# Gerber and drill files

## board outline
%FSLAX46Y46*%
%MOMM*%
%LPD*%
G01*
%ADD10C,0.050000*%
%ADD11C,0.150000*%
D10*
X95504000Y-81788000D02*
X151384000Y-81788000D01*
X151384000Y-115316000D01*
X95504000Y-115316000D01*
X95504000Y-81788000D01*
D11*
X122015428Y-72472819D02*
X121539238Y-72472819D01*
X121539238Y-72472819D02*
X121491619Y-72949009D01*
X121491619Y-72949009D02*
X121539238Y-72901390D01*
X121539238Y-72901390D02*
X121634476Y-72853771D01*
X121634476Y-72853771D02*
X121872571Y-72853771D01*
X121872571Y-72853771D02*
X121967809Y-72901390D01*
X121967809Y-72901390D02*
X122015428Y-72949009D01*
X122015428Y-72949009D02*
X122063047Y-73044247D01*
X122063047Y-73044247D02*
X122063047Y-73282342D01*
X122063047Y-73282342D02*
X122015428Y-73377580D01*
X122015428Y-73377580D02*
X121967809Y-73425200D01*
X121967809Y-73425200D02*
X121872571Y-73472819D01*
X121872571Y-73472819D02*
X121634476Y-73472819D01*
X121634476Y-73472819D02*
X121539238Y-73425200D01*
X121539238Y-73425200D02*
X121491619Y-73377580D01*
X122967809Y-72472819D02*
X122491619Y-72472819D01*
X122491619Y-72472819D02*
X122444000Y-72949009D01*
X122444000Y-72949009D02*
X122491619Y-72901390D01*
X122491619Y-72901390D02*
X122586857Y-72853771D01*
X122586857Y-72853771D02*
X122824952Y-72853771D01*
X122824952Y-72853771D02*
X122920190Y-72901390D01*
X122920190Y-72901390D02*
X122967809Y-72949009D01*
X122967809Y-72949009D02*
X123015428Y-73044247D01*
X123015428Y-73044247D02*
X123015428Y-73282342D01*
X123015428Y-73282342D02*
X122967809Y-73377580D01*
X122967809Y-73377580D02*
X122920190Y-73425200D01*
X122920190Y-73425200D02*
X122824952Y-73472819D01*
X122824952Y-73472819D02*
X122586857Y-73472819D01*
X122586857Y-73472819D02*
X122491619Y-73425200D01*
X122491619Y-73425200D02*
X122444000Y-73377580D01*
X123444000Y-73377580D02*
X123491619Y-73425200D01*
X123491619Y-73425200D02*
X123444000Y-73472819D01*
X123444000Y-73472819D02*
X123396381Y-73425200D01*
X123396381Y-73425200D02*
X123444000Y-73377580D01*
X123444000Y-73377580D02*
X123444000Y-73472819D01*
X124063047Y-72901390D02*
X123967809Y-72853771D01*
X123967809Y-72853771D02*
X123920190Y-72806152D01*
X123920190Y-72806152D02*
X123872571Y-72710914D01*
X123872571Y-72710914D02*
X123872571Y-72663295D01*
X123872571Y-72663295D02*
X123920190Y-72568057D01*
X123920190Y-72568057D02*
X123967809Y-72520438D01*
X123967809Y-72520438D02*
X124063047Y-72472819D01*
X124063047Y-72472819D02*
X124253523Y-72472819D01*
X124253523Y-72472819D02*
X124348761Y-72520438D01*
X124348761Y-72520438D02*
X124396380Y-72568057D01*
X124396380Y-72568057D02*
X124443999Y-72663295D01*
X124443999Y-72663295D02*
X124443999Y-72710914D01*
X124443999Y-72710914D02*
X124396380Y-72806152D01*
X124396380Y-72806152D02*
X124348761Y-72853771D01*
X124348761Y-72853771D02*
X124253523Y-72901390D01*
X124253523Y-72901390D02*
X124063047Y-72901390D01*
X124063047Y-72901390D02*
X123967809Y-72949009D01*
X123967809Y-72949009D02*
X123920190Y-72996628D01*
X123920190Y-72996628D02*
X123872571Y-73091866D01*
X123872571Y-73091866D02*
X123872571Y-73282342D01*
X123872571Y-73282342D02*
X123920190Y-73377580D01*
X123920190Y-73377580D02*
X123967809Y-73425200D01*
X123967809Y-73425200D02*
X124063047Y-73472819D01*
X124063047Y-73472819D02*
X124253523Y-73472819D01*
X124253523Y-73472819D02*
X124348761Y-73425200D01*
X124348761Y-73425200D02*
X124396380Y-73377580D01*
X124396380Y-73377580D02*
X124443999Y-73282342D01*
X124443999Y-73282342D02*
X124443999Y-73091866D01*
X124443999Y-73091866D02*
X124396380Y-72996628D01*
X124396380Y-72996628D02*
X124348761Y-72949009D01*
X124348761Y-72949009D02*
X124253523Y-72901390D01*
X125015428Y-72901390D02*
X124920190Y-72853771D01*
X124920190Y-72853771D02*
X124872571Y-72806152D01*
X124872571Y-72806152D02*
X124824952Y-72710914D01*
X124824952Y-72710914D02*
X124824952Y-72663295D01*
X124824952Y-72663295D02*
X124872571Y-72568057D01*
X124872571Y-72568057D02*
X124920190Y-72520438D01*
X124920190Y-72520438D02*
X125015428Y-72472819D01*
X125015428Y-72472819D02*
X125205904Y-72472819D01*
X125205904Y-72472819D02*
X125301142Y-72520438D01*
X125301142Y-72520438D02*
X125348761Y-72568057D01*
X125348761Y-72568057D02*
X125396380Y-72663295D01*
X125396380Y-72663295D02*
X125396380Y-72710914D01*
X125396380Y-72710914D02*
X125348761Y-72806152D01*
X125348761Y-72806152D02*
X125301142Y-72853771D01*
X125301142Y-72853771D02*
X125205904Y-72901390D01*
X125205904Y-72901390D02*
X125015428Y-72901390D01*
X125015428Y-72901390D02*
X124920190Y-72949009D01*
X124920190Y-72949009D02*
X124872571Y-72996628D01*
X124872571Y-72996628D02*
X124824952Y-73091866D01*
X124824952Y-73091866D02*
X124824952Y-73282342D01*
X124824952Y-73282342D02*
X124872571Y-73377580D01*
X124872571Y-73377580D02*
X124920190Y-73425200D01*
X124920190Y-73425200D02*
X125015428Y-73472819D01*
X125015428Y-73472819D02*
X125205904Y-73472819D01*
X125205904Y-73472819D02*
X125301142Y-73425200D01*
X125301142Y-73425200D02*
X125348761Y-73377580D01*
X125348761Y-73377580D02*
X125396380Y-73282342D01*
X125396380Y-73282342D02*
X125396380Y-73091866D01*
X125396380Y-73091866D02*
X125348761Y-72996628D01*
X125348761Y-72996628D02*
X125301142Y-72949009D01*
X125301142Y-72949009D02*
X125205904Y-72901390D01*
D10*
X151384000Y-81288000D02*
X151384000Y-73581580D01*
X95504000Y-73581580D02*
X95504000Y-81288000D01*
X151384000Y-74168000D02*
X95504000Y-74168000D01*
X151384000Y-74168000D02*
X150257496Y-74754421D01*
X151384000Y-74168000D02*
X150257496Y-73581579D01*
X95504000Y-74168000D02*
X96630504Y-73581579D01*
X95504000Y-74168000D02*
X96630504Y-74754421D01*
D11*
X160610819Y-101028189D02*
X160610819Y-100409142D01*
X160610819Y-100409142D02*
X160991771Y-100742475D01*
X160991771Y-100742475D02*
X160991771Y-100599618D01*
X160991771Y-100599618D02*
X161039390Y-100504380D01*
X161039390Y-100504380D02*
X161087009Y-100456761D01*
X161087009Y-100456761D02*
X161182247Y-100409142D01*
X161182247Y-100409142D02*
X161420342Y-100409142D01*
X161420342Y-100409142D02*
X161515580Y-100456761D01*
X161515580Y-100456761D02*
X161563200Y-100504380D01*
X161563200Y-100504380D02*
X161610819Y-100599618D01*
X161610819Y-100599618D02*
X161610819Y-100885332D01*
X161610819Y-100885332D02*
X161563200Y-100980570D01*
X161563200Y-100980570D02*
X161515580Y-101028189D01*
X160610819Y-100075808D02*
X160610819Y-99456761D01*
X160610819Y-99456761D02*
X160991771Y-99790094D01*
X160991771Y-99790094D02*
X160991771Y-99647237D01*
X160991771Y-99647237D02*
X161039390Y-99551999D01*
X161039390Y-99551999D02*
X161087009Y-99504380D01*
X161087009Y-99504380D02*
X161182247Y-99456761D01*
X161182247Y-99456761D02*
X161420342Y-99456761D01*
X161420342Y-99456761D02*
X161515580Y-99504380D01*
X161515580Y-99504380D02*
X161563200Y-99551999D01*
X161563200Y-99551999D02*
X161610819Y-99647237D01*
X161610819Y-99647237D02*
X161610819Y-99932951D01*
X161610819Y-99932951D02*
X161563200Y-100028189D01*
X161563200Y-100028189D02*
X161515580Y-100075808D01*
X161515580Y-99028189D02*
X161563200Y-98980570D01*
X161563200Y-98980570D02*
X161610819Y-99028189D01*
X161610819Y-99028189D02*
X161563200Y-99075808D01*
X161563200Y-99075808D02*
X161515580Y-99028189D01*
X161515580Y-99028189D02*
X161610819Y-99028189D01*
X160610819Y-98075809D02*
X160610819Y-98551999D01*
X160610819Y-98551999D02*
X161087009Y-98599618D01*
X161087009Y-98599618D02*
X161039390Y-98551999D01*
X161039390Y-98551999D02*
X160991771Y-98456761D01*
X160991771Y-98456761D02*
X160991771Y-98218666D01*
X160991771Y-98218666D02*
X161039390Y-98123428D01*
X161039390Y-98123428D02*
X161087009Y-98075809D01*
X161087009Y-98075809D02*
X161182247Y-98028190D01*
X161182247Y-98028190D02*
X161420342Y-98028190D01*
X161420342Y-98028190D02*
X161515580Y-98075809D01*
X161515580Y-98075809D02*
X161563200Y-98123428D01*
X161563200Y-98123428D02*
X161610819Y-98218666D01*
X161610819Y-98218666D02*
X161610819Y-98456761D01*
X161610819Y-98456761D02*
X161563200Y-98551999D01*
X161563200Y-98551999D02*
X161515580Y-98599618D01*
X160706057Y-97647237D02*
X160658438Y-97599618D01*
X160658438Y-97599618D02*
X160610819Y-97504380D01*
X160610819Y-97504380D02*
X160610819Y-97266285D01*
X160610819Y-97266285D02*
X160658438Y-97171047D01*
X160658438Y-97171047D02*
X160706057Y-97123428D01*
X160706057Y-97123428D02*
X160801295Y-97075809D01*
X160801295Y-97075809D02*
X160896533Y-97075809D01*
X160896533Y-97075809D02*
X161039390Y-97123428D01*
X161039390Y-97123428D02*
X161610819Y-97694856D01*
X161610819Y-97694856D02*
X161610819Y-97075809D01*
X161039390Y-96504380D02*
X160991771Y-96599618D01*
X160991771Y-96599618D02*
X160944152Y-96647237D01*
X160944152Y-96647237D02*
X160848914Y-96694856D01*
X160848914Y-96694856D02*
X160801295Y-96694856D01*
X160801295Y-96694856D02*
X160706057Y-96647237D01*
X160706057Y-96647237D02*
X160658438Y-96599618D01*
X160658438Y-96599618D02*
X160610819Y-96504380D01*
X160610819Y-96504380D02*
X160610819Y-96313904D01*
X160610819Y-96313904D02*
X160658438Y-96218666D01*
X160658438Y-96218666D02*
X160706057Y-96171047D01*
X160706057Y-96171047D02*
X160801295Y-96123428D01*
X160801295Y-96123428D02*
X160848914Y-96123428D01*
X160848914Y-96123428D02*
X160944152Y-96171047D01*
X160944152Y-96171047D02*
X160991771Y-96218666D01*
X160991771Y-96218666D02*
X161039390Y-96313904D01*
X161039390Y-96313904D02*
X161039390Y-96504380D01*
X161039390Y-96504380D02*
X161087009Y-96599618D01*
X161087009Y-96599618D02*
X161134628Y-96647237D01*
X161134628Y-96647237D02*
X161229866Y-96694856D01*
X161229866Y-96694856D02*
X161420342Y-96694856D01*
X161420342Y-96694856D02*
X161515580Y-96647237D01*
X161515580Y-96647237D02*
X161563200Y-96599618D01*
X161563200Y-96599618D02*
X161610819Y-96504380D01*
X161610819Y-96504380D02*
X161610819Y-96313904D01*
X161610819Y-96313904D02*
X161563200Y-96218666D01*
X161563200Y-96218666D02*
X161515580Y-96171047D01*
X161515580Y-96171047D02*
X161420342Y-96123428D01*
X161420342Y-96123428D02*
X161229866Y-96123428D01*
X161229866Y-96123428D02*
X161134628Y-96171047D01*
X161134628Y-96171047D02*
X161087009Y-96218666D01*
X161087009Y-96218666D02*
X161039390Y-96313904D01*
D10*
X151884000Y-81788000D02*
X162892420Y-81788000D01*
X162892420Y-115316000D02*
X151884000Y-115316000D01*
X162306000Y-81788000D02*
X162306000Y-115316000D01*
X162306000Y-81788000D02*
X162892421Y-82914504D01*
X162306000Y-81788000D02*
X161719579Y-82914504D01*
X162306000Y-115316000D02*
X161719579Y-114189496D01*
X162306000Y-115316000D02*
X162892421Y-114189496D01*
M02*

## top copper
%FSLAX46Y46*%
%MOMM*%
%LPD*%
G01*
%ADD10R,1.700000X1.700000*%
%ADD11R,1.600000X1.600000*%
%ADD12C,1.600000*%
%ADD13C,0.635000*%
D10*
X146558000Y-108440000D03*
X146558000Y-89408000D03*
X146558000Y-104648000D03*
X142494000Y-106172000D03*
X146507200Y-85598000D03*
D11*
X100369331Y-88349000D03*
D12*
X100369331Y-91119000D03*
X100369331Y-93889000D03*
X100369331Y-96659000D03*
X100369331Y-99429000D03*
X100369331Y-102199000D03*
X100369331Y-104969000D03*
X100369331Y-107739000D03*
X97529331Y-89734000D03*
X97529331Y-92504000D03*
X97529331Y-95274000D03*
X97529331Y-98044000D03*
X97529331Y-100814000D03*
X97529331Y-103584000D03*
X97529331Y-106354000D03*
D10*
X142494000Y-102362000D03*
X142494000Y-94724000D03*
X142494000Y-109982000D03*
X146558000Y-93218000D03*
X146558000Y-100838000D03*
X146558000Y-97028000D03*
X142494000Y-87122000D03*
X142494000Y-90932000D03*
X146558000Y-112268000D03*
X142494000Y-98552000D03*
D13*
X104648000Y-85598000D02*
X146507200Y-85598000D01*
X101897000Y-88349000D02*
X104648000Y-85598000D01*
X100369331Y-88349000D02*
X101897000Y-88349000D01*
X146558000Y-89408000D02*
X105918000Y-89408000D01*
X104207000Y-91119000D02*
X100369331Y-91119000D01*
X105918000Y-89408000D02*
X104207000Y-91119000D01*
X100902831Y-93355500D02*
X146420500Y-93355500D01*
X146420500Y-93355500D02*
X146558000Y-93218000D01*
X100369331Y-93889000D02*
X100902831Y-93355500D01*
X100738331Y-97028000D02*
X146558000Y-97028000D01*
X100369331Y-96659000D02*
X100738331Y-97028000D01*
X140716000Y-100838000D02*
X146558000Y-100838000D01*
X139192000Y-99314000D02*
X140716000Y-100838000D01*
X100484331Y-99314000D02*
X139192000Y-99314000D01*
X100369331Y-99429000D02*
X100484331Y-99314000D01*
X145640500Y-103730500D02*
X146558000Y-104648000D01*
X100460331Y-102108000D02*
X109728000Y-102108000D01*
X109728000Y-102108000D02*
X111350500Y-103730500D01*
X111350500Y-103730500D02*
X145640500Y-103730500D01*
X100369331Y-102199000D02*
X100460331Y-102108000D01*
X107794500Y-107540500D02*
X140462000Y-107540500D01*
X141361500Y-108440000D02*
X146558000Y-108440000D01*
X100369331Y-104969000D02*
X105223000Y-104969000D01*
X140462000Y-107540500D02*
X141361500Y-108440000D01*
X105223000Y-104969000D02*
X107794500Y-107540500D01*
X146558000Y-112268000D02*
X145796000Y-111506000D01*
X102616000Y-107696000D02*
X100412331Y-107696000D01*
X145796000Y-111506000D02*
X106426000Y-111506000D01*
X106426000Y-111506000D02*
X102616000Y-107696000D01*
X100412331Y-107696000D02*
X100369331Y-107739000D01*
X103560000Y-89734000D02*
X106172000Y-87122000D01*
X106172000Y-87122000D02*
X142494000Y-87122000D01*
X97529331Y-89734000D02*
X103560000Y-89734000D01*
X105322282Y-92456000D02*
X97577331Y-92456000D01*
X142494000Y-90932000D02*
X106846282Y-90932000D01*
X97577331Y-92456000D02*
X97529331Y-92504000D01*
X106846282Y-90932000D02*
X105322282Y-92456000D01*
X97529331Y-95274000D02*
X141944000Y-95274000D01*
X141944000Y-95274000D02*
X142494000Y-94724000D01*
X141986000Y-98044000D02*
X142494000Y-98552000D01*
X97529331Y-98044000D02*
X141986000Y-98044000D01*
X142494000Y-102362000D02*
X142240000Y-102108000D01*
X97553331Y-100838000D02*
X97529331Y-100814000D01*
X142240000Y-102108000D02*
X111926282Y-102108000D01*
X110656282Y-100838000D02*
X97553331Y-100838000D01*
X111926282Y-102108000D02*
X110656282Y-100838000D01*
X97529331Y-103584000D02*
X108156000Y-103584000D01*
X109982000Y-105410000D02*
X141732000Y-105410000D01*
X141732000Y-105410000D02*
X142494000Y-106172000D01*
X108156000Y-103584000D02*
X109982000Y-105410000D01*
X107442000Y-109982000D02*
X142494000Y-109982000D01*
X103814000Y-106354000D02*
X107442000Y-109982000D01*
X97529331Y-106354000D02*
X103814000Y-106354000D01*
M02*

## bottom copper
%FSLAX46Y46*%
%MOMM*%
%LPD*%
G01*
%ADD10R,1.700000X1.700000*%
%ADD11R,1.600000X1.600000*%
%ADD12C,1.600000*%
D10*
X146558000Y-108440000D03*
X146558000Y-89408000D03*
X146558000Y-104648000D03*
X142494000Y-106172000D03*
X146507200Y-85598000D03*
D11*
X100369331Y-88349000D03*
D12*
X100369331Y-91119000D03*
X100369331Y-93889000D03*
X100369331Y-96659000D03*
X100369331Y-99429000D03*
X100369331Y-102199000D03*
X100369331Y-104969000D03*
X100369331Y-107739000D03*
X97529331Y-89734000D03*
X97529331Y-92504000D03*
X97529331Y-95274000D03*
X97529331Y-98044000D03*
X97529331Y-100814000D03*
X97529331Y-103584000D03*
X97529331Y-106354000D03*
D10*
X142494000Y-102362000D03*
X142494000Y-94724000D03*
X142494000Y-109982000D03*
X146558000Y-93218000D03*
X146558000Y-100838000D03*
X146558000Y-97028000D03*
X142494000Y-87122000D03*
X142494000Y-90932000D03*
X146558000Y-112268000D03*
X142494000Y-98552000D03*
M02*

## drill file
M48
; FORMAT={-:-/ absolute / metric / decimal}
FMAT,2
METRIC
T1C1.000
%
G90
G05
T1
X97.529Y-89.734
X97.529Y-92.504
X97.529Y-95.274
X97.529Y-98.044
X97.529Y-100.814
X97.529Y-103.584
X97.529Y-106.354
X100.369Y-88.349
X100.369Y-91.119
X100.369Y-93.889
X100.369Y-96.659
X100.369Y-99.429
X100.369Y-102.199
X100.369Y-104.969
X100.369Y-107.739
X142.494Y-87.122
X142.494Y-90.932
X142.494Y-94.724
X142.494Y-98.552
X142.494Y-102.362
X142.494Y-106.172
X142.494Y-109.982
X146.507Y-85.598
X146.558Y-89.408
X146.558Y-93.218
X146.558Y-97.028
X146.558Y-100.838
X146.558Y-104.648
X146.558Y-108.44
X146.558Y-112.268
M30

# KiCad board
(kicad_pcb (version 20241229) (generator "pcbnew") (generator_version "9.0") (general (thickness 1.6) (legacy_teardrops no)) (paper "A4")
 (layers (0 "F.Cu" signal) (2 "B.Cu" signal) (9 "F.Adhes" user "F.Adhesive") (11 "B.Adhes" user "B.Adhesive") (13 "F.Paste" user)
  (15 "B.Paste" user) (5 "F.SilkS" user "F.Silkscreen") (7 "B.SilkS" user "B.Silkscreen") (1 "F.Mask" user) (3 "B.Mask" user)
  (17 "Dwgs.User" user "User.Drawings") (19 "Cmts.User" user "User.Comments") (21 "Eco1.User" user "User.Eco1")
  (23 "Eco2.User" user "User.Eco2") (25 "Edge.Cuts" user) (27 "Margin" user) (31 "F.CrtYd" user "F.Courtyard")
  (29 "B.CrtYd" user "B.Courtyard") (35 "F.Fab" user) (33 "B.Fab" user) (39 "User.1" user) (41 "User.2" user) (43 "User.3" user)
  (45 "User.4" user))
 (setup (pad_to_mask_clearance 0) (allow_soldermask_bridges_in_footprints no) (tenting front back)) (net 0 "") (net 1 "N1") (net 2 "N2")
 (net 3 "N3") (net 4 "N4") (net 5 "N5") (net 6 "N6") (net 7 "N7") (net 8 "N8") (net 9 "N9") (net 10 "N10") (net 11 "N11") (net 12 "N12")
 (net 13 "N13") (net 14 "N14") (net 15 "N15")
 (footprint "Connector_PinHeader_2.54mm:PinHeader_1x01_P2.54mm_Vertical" (layer "F.Cu") (at 146.558 108.44)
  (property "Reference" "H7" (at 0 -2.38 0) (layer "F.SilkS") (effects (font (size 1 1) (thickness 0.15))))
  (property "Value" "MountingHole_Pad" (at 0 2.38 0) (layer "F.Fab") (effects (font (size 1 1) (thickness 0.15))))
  (pad "1" thru_hole rect (at 0 0) (size 1.7 1.7) (drill 1) (layers "*.Cu" "*.Mask") (remove_unused_layers no) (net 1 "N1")))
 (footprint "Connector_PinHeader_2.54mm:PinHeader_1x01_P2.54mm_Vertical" (layer "F.Cu") (at 146.558 89.408)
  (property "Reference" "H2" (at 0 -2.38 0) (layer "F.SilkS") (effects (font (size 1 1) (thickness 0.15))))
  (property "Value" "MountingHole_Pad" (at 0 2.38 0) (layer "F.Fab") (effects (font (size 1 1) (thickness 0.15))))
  (pad "1" thru_hole rect (at 0 0) (size 1.7 1.7) (drill 1) (layers "*.Cu" "*.Mask") (remove_unused_layers no) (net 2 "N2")))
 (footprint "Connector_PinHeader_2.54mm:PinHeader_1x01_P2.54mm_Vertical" (layer "F.Cu") (at 146.558 104.648)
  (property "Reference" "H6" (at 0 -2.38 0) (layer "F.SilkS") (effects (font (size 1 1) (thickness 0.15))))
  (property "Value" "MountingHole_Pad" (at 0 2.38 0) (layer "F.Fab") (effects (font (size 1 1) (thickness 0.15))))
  (pad "1" thru_hole rect (at 0 0) (size 1.7 1.7) (drill 1) (layers "*.Cu" "*.Mask") (remove_unused_layers no) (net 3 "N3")))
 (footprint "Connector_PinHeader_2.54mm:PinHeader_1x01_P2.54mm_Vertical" (layer "F.Cu") (at 142.494 106.172)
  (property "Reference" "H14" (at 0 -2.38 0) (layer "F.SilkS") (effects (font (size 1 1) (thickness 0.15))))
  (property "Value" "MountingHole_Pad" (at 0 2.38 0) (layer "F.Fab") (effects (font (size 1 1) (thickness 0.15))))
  (pad "1" thru_hole rect (at 0 0) (size 1.7 1.7) (drill 1) (layers "*.Cu" "*.Mask") (remove_unused_layers no) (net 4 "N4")))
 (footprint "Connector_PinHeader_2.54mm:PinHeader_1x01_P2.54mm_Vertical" (layer "F.Cu") (at 146.5072 85.598)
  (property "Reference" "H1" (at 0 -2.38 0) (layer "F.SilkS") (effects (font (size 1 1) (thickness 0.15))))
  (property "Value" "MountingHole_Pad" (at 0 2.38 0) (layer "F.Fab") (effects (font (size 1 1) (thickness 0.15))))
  (pad "1" thru_hole rect (at 0 0) (size 1.7 1.7) (drill 1) (layers "*.Cu" "*.Mask") (remove_unused_layers no) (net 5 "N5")))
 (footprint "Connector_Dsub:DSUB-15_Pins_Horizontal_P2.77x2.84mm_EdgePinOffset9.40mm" (layer "F.Cu") (at 100.369331 88.349 -90)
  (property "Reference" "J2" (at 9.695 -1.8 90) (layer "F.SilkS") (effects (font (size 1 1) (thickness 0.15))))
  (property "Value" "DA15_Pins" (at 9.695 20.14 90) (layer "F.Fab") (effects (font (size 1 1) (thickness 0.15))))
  (pad "1" thru_hole rect (at 0 0 270) (size 1.6 1.6) (drill 1) (layers "*.Cu" "*.Mask") (remove_unused_layers no) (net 5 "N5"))
  (pad "2" thru_hole circle (at 2.77 0 270) (size 1.6 1.6) (drill 1) (layers "*.Cu" "*.Mask") (remove_unused_layers no) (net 2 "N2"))
  (pad "3" thru_hole circle (at 5.54 0 270) (size 1.6 1.6) (drill 1) (layers "*.Cu" "*.Mask") (remove_unused_layers no) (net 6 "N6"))
  (pad "4" thru_hole circle (at 8.31 0 270) (size 1.6 1.6) (drill 1) (layers "*.Cu" "*.Mask") (remove_unused_layers no) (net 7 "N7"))
  (pad "5" thru_hole circle (at 11.08 0 270) (size 1.6 1.6) (drill 1) (layers "*.Cu" "*.Mask") (remove_unused_layers no) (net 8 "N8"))
  (pad "6" thru_hole circle (at 13.85 0 270) (size 1.6 1.6) (drill 1) (layers "*.Cu" "*.Mask") (remove_unused_layers no) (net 3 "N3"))
  (pad "7" thru_hole circle (at 16.62 0 270) (size 1.6 1.6) (drill 1) (layers "*.Cu" "*.Mask") (remove_unused_layers no) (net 1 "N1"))
  (pad "8" thru_hole circle (at 19.39 0 270) (size 1.6 1.6) (drill 1) (layers "*.Cu" "*.Mask") (remove_unused_layers no) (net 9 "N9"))
  (pad "9" thru_hole circle (at 1.385 2.84 270) (size 1.6 1.6) (drill 1) (layers "*.Cu" "*.Mask") (remove_unused_layers no) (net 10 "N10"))
  (pad "10" thru_hole circle (at 4.155 2.84 270) (size 1.6 1.6) (drill 1) (layers "*.Cu" "*.Mask") (remove_unused_layers no) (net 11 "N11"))
  (pad "11" thru_hole circle (at 6.925 2.84 270) (size 1.6 1.6) (drill 1) (layers "*.Cu" "*.Mask") (remove_unused_layers no) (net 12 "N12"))
  (pad "12" thru_hole circle (at 9.695 2.84 270) (size 1.6 1.6) (drill 1) (layers "*.Cu" "*.Mask") (remove_unused_layers no) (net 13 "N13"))
  (pad "13" thru_hole circle (at 12.465 2.84 270) (size 1.6 1.6) (drill 1) (layers "*.Cu" "*.Mask") (remove_unused_layers no) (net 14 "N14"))
  (pad "14" thru_hole circle (at 15.235 2.84 270) (size 1.6 1.6) (drill 1) (layers "*.Cu" "*.Mask") (remove_unused_layers no) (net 4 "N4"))
  (pad "15" thru_hole circle (at 18.005 2.84 270) (size 1.6 1.6) (drill 1) (layers "*.Cu" "*.Mask") (remove_unused_layers no) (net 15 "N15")))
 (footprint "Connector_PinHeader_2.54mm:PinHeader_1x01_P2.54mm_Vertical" (layer "F.Cu") (at 142.494 102.362)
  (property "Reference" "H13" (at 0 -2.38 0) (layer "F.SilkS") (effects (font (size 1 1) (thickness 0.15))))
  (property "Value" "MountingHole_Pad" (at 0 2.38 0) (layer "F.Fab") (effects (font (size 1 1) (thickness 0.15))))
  (pad "1" thru_hole rect (at 0 0) (size 1.7 1.7) (drill 1) (layers "*.Cu" "*.Mask") (remove_unused_layers no) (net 14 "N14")))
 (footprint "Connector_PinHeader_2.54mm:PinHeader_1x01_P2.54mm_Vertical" (layer "F.Cu") (at 142.494 94.724)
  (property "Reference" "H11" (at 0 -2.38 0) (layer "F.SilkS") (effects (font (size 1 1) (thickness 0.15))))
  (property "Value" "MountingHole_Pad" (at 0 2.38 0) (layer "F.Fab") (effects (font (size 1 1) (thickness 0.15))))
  (pad "1" thru_hole rect (at 0 0) (size 1.7 1.7) (drill 1) (layers "*.Cu" "*.Mask") (remove_unused_layers no) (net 12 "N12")))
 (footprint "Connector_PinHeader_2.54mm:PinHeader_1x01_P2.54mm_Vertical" (layer "F.Cu") (at 142.494 109.982)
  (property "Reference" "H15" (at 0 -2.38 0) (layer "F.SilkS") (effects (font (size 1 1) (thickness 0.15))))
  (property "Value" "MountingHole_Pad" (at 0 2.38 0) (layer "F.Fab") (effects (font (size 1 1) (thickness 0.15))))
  (pad "1" thru_hole rect (at 0 0) (size 1.7 1.7) (drill 1) (layers "*.Cu" "*.Mask") (remove_unused_layers no) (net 15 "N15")))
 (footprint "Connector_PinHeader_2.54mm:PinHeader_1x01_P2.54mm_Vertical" (layer "F.Cu") (at 146.558 93.218)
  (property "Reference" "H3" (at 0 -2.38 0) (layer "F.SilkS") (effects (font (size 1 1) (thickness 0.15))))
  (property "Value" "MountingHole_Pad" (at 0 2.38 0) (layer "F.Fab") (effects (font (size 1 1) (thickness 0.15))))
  (pad "1" thru_hole rect (at 0 0) (size 1.7 1.7) (drill 1) (layers "*.Cu" "*.Mask") (remove_unused_layers no) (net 6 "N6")))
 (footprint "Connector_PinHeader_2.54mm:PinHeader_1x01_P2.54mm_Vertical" (layer "F.Cu") (at 146.558 100.838)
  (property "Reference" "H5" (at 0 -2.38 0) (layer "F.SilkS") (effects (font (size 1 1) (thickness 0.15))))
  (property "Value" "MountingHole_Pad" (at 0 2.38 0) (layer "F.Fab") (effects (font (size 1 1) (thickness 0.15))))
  (pad "1" thru_hole rect (at 0 0) (size 1.7 1.7) (drill 1) (layers "*.Cu" "*.Mask") (remove_unused_layers no) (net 8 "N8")))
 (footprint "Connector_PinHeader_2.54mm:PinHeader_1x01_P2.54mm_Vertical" (layer "F.Cu") (at 146.558 97.028)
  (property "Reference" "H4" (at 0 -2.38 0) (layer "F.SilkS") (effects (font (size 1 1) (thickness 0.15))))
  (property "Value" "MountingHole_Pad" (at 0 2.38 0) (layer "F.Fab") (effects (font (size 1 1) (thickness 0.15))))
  (pad "1" thru_hole rect (at 0 0) (size 1.7 1.7) (drill 1) (layers "*.Cu" "*.Mask") (remove_unused_layers no) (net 7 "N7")))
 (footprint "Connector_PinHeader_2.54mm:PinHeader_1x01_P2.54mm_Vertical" (layer "F.Cu") (at 142.494 87.122)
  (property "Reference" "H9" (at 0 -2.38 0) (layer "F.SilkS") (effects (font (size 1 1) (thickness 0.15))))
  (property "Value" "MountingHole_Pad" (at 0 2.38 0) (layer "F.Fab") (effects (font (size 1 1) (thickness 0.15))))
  (pad "1" thru_hole rect (at 0 0) (size 1.7 1.7) (drill 1) (layers "*.Cu" "*.Mask") (remove_unused_layers no) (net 10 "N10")))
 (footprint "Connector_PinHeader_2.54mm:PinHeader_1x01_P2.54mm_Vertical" (layer "F.Cu") (at 142.494 90.932)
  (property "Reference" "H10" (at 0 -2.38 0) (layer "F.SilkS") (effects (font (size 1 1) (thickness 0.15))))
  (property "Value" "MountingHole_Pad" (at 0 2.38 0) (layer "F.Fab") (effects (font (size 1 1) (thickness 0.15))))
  (pad "1" thru_hole rect (at 0 0) (size 1.7 1.7) (drill 1) (layers "*.Cu" "*.Mask") (remove_unused_layers no) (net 11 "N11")))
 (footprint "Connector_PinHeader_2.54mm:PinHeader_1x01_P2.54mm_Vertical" (layer "F.Cu") (at 146.558 112.268)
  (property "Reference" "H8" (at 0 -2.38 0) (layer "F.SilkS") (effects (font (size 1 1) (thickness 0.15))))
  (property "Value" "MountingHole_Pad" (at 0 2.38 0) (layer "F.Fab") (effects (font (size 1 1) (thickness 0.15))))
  (pad "1" thru_hole rect (at 0 0) (size 1.7 1.7) (drill 1) (layers "*.Cu" "*.Mask") (remove_unused_layers no) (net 9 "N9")))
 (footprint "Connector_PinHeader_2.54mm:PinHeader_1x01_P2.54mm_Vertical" (layer "F.Cu") (at 142.494 98.552)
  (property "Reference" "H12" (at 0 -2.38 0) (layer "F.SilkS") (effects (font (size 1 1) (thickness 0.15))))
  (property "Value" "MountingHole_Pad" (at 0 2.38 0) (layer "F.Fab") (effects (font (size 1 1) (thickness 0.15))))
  (pad "1" thru_hole rect (at 0 0) (size 1.7 1.7) (drill 1) (layers "*.Cu" "*.Mask") (remove_unused_layers no) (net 13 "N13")))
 (gr_rect (start 95.504 81.788) (end 151.384 115.316) (stroke (width 0.05) (type default)) (fill no) (layer "Edge.Cuts"))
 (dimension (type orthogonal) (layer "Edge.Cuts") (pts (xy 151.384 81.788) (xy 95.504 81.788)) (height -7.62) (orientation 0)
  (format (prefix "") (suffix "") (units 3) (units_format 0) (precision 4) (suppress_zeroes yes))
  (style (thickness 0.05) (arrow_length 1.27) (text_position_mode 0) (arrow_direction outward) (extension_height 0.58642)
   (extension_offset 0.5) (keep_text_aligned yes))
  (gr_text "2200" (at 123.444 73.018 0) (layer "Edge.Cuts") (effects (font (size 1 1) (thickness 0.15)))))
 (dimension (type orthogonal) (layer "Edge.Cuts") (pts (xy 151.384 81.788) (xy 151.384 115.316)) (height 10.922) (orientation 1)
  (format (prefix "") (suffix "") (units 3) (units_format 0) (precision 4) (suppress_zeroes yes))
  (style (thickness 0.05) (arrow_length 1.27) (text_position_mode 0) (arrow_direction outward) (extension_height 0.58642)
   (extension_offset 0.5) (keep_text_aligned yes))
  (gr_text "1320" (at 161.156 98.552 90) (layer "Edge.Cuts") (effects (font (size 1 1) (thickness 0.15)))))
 (segment (start 104.648 85.598) (end 146.5072 85.598) (width 0.635) (layer "F.Cu") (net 5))
 (segment (start 101.897 88.349) (end 104.648 85.598) (width 0.635) (layer "F.Cu") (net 5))
 (segment (start 100.369331 88.349) (end 101.897 88.349) (width 0.635) (layer "F.Cu") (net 5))
 (segment (start 146.558 89.408) (end 105.918 89.408) (width 0.635) (layer "F.Cu") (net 2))
 (segment (start 104.207 91.119) (end 100.369331 91.119) (width 0.635) (layer "F.Cu") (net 2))
 (segment (start 105.918 89.408) (end 104.207 91.119) (width 0.635) (layer "F.Cu") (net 2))
 (segment (start 100.902831 93.3555) (end 146.4205 93.3555) (width 0.635) (layer "F.Cu") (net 6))
 (segment (start 146.4205 93.3555) (end 146.558 93.218) (width 0.635) (layer "F.Cu") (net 6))
 (segment (start 100.369331 93.889) (end 100.902831 93.3555) (width 0.635) (layer "F.Cu") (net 6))
 (segment (start 100.738331 97.028) (end 146.558 97.028) (width 0.635) (layer "F.Cu") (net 7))
 (segment (start 100.369331 96.659) (end 100.738331 97.028) (width 0.635) (layer "F.Cu") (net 7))
 (segment (start 140.716 100.838) (end 146.558 100.838) (width 0.635) (layer "F.Cu") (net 8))
 (segment (start 139.192 99.314) (end 140.716 100.838) (width 0.635) (layer "F.Cu") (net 8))
 (segment (start 100.484331 99.314) (end 139.192 99.314) (width 0.635) (layer "F.Cu") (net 8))
 (segment (start 100.369331 99.429) (end 100.484331 99.314) (width 0.635) (layer "F.Cu") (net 8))
 (segment (start 145.6405 103.7305) (end 146.558 104.648) (width 0.635) (layer "F.Cu") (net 3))
 (segment (start 100.460331 102.108) (end 109.728 102.108) (width 0.635) (layer "F.Cu") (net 3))
 (segment (start 109.728 102.108) (end 111.3505 103.7305) (width 0.635) (layer "F.Cu") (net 3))
 (segment (start 111.3505 103.7305) (end 145.6405 103.7305) (width 0.635) (layer "F.Cu") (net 3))
 (segment (start 100.369331 102.199) (end 100.460331 102.108) (width 0.635) (layer "F.Cu") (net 3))
 (segment (start 107.7945 107.5405) (end 140.462 107.5405) (width 0.635) (layer "F.Cu") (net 1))
 (segment (start 141.3615 108.44) (end 146.558 108.44) (width 0.635) (layer "F.Cu") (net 1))
 (segment (start 100.369331 104.969) (end 105.223 104.969) (width 0.635) (layer "F.Cu") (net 1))
 (segment (start 140.462 107.5405) (end 141.3615 108.44) (width 0.635) (layer "F.Cu") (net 1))
 (segment (start 105.223 104.969) (end 107.7945 107.5405) (width 0.635) (layer "F.Cu") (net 1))
 (segment (start 146.558 112.268) (end 145.796 111.506) (width 0.635) (layer "F.Cu") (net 9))
 (segment (start 102.616 107.696) (end 100.412331 107.696) (width 0.635) (layer "F.Cu") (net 9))
 (segment (start 145.796 111.506) (end 106.426 111.506) (width 0.635) (layer "F.Cu") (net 9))
 (segment (start 106.426 111.506) (end 102.616 107.696) (width 0.635) (layer "F.Cu") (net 9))
 (segment (start 100.412331 107.696) (end 100.369331 107.739) (width 0.635) (layer "F.Cu") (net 9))
 (segment (start 103.56 89.734) (end 106.172 87.122) (width 0.635) (layer "F.Cu") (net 10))
 (segment (start 106.172 87.122) (end 142.494 87.122) (width 0.635) (layer "F.Cu") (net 10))
 (segment (start 97.529331 89.734) (end 103.56 89.734) (width 0.635) (layer "F.Cu") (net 10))
 (segment (start 105.322282 92.456) (end 97.577331 92.456) (width 0.635) (layer "F.Cu") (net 11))
 (segment (start 142.494 90.932) (end 106.846282 90.932) (width 0.635) (layer "F.Cu") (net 11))
 (segment (start 97.577331 92.456) (end 97.529331 92.504) (width 0.635) (layer "F.Cu") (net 11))
 (segment (start 106.846282 90.932) (end 105.322282 92.456) (width 0.635) (layer "F.Cu") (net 11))
 (segment (start 97.529331 95.274) (end 141.944 95.274) (width 0.635) (layer "F.Cu") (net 12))
 (segment (start 141.944 95.274) (end 142.494 94.724) (width 0.635) (layer "F.Cu") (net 12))
 (segment (start 141.986 98.044) (end 142.494 98.552) (width 0.635) (layer "F.Cu") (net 13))
 (segment (start 97.529331 98.044) (end 141.986 98.044) (width 0.635) (layer "F.Cu") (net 13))
 (segment (start 142.494 102.362) (end 142.24 102.108) (width 0.635) (layer "F.Cu") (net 14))
 (segment (start 97.553331 100.838) (end 97.529331 100.814) (width 0.635) (layer "F.Cu") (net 14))
 (segment (start 142.24 102.108) (end 111.926282 102.108) (width 0.635) (layer "F.Cu") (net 14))
 (segment (start 110.656282 100.838) (end 97.553331 100.838) (width 0.635) (layer "F.Cu") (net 14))
 (segment (start 111.926282 102.108) (end 110.656282 100.838) (width 0.635) (layer "F.Cu") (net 14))
 (segment (start 97.529331 103.584) (end 108.156 103.584) (width 0.635) (layer "F.Cu") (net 4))
 (segment (start 109.982 105.41) (end 141.732 105.41) (width 0.635) (layer "F.Cu") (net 4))
 (segment (start 141.732 105.41) (end 142.494 106.172) (width 0.635) (layer "F.Cu") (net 4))
 (segment (start 108.156 103.584) (end 109.982 105.41) (width 0.635) (layer "F.Cu") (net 4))
 (segment (start 107.442 109.982) (end 142.494 109.982) (width 0.635) (layer "F.Cu") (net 15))
 (segment (start 103.814 106.354) (end 107.442 109.982) (width 0.635) (layer "F.Cu") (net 15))
 (segment (start 97.529331 106.354) (end 103.814 106.354) (width 0.635) (layer "F.Cu") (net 15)))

